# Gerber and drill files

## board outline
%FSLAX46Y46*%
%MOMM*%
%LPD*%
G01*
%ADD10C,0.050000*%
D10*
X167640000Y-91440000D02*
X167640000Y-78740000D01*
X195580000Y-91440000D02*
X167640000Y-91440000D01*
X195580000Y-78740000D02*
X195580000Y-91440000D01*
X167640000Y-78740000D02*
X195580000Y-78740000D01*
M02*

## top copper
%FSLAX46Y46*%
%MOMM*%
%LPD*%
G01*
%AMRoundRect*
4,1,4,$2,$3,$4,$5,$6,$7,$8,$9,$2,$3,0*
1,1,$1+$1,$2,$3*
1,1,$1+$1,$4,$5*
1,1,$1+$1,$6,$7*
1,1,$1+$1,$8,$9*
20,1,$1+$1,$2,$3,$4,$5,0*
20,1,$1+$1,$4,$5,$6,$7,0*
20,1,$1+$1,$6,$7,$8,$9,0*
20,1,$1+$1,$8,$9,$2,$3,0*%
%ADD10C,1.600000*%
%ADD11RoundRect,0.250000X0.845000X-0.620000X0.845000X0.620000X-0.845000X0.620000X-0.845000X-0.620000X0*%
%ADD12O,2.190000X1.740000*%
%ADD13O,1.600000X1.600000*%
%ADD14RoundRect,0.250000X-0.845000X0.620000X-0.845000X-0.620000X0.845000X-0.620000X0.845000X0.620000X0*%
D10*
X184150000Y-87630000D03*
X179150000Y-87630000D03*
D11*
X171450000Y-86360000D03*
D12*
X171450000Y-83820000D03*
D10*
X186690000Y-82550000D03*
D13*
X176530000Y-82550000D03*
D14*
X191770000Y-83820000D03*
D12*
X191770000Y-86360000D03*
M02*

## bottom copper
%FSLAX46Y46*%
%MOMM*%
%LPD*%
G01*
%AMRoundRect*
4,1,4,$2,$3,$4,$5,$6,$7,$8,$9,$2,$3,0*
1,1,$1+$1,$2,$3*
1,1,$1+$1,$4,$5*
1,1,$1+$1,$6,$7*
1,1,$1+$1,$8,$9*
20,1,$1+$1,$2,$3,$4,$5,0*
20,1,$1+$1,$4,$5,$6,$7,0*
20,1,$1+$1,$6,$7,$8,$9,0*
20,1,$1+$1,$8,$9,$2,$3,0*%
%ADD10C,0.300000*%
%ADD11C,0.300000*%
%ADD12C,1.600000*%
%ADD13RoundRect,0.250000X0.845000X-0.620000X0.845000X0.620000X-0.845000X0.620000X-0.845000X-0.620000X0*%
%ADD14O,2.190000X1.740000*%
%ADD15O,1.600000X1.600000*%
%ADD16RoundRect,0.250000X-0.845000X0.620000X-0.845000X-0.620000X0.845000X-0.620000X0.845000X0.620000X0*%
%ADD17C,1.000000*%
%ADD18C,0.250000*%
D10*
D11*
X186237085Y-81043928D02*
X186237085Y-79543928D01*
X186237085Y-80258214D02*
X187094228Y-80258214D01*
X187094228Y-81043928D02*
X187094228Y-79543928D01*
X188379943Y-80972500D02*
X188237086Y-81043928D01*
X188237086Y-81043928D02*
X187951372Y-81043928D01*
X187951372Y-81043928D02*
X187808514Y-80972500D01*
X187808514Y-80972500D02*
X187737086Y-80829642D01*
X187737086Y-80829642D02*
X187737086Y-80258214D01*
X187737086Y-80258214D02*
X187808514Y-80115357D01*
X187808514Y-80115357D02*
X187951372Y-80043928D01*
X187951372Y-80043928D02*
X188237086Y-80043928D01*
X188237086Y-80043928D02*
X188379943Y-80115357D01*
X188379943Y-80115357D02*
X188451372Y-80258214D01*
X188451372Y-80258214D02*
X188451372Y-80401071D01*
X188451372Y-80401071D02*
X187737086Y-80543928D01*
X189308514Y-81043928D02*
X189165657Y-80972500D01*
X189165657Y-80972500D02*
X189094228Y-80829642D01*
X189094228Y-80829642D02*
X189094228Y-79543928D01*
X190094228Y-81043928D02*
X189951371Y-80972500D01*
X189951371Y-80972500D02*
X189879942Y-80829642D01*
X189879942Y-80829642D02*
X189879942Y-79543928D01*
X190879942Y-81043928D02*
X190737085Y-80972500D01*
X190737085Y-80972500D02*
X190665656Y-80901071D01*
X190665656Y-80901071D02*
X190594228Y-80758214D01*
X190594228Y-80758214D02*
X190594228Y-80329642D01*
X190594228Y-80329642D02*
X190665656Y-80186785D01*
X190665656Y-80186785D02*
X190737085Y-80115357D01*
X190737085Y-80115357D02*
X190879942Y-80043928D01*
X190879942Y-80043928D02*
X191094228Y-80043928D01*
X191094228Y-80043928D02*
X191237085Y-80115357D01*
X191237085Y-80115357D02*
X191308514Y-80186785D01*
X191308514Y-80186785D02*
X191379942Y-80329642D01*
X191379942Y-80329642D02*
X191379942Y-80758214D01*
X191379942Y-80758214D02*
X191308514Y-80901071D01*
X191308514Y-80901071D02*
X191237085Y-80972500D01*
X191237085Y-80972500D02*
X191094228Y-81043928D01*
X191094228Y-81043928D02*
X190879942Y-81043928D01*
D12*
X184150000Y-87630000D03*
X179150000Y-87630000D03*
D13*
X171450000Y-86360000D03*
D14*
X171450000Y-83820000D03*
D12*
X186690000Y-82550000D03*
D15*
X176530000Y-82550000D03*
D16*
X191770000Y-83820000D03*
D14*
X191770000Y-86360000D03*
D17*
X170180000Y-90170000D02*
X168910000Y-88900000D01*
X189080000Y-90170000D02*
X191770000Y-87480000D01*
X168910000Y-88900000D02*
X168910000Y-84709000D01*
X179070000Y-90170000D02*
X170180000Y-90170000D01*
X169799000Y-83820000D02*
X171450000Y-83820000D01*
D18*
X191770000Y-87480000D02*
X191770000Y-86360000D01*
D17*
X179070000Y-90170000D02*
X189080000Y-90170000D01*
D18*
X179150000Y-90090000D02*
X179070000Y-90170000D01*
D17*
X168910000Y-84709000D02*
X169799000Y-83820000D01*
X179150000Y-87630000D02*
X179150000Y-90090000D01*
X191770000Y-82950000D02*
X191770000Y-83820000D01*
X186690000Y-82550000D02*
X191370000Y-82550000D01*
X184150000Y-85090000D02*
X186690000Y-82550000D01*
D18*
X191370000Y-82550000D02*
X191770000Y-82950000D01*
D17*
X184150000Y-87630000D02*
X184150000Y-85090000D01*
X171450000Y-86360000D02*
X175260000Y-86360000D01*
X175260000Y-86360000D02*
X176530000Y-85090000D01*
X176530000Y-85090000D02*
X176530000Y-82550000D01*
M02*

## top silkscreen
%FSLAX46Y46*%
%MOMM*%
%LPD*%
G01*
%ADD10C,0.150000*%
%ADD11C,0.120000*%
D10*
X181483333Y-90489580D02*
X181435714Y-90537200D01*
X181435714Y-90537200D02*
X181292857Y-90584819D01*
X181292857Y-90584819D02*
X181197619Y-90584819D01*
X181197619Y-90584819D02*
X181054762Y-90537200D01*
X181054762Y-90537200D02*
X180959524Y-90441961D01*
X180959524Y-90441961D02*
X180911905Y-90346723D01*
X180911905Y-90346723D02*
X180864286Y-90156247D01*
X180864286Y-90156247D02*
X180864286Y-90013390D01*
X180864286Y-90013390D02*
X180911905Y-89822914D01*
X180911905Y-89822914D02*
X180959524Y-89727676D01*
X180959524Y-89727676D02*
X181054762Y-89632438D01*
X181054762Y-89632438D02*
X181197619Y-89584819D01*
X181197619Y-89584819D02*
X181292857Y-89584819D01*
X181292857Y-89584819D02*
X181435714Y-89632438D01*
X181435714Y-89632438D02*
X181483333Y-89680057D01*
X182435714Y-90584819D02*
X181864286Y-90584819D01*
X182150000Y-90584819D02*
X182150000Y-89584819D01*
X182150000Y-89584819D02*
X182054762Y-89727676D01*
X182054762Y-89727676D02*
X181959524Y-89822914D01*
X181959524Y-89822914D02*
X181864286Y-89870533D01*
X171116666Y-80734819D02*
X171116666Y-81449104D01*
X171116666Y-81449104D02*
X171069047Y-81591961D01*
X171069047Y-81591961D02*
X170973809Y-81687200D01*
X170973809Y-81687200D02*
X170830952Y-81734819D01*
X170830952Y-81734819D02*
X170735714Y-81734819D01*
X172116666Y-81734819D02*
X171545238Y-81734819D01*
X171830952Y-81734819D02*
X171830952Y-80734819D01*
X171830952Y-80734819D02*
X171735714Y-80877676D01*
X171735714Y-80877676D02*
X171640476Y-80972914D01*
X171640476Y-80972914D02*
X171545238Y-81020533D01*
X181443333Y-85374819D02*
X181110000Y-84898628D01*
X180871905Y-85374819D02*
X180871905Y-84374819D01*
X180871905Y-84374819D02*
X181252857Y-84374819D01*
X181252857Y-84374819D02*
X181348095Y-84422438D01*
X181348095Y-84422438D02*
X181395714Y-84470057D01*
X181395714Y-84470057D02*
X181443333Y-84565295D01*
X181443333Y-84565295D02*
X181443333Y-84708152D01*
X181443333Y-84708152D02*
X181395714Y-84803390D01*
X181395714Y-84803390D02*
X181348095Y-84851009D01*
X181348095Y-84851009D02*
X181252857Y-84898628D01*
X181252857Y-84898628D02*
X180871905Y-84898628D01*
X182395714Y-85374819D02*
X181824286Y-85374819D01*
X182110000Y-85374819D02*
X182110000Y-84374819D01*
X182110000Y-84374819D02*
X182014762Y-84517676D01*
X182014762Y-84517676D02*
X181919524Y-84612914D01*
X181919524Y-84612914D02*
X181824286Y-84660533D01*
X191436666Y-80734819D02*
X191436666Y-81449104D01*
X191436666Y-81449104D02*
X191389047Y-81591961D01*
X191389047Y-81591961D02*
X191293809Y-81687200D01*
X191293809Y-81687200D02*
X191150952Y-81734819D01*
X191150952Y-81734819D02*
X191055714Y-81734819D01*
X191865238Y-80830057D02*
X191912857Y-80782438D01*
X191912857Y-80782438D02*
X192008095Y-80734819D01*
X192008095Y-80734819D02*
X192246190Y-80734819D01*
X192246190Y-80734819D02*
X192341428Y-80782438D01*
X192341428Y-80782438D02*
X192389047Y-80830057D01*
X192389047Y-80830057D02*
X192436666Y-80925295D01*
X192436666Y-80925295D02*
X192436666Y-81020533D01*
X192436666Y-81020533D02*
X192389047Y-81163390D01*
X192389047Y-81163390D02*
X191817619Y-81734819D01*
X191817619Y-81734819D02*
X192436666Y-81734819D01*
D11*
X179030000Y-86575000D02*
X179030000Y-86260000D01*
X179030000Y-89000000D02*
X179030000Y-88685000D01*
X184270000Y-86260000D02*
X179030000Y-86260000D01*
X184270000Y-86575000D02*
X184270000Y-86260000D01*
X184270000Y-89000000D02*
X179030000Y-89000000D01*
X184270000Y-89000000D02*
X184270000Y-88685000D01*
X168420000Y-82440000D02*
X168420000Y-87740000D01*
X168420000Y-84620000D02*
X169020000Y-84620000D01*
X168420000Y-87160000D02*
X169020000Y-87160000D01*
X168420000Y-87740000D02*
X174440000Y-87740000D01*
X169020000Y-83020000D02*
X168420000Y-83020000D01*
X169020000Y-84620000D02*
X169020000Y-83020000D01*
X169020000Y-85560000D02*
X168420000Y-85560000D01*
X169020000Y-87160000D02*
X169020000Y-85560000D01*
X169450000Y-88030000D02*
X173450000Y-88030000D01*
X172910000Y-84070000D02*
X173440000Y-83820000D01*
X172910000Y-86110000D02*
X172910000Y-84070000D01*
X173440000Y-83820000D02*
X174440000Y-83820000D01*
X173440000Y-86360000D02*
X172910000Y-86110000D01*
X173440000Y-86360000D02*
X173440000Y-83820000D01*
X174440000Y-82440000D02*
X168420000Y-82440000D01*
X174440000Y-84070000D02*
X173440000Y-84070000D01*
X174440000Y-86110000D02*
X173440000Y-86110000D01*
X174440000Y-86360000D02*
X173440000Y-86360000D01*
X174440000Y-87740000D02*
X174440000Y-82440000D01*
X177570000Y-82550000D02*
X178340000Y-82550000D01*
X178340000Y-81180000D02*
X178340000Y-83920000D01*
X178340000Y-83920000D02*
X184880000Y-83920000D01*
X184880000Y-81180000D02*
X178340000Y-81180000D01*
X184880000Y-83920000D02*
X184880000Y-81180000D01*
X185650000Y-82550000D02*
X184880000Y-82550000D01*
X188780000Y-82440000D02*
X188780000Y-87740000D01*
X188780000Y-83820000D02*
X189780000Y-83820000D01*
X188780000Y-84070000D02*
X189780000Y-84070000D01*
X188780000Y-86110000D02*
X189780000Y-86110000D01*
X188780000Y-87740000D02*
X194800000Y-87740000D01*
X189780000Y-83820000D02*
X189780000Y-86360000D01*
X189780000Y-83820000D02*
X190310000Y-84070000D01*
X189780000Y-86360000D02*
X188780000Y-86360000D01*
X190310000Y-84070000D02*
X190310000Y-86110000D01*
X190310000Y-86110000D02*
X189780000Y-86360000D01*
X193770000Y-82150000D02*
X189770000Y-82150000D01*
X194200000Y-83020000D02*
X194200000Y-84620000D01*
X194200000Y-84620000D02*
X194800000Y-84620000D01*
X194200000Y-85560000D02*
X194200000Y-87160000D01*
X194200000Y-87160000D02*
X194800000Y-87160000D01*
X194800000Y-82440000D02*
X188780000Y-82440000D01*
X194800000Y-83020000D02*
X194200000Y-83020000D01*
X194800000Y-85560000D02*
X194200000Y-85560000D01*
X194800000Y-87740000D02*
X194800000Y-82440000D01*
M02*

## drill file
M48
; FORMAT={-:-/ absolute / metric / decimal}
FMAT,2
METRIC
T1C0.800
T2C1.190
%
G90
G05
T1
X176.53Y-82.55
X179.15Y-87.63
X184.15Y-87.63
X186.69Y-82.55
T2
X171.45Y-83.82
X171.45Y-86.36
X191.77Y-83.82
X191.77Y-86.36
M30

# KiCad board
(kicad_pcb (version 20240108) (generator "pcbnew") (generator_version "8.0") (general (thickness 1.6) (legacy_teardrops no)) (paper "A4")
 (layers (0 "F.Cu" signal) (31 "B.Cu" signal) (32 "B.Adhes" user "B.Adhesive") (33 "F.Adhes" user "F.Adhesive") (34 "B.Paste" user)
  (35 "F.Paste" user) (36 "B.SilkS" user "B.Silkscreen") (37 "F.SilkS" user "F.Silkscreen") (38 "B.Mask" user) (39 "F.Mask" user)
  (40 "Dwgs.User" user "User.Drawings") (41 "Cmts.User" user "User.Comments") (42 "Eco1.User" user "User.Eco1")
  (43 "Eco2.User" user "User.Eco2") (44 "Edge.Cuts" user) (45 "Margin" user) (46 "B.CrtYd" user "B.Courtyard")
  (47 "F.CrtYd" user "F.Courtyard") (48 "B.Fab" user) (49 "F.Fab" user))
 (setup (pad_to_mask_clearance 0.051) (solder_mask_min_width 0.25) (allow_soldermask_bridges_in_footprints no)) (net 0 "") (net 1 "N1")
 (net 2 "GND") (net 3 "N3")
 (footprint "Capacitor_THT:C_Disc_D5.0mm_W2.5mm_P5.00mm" (layer "F.Cu") (at 184.15 87.63 180)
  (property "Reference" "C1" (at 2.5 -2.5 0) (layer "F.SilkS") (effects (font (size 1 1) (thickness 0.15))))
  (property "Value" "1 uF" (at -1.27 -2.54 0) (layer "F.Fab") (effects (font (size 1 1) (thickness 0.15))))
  (fp_line (start 5.12 1.055) (end 5.12 1.37) (stroke (width 0.12) (type solid)) (layer "F.SilkS"))
  (fp_line (start 5.12 -1.37) (end 5.12 -1.055) (stroke (width 0.12) (type solid)) (layer "F.SilkS"))
  (fp_line (start -0.12 1.37) (end 5.12 1.37) (stroke (width 0.12) (type solid)) (layer "F.SilkS"))
  (fp_line (start -0.12 1.055) (end -0.12 1.37) (stroke (width 0.12) (type solid)) (layer "F.SilkS"))
  (fp_line (start -0.12 -1.37) (end 5.12 -1.37) (stroke (width 0.12) (type solid)) (layer "F.SilkS"))
  (fp_line (start -0.12 -1.37) (end -0.12 -1.055) (stroke (width 0.12) (type solid)) (layer "F.SilkS"))
  (pad "1" thru_hole circle (at 0 0 180) (size 1.6 1.6) (drill 0.8) (layers "*.Cu" "*.Mask") (remove_unused_layers no) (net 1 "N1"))
  (pad "2" thru_hole circle (at 5 0 180) (size 1.6 1.6) (drill 0.8) (layers "*.Cu" "*.Mask") (remove_unused_layers no) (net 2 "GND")))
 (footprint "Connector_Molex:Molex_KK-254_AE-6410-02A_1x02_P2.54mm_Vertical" (layer "F.Cu") (at 171.45 86.36 90)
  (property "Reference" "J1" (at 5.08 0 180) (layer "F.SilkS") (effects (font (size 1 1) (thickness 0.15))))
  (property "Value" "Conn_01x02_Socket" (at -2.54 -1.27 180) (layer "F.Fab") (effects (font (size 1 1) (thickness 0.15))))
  (fp_line (start 3.92 -3.03) (end -1.38 -3.03) (stroke (width 0.12) (type solid)) (layer "F.SilkS"))
  (fp_line (start 1.74 -3.03) (end 1.74 -2.43) (stroke (width 0.12) (type solid)) (layer "F.SilkS"))
  (fp_line (start -0.8 -3.03) (end -0.8 -2.43) (stroke (width 0.12) (type solid)) (layer "F.SilkS"))
  (fp_line (start -1.38 -3.03) (end -1.38 2.99) (stroke (width 0.12) (type solid)) (layer "F.SilkS"))
  (fp_line (start 3.34 -2.43) (end 3.34 -3.03) (stroke (width 0.12) (type solid)) (layer "F.SilkS"))
  (fp_line (start 1.74 -2.43) (end 3.34 -2.43) (stroke (width 0.12) (type solid)) (layer "F.SilkS"))
  (fp_line (start 0.8 -2.43) (end 0.8 -3.03) (stroke (width 0.12) (type solid)) (layer "F.SilkS"))
  (fp_line (start -0.8 -2.43) (end 0.8 -2.43) (stroke (width 0.12) (type solid)) (layer "F.SilkS"))
  (fp_line (start -1.67 -2) (end -1.67 2) (stroke (width 0.12) (type solid)) (layer "F.SilkS"))
  (fp_line (start 2.29 1.46) (end 2.54 1.99) (stroke (width 0.12) (type solid)) (layer "F.SilkS"))
  (fp_line (start 0.25 1.46) (end 2.29 1.46) (stroke (width 0.12) (type solid)) (layer "F.SilkS"))
  (fp_line (start 2.54 1.99) (end 2.54 2.99) (stroke (width 0.12) (type solid)) (layer "F.SilkS"))
  (fp_line (start 0 1.99) (end 0.25 1.46) (stroke (width 0.12) (type solid)) (layer "F.SilkS"))
  (fp_line (start 0 1.99) (end 2.54 1.99) (stroke (width 0.12) (type solid)) (layer "F.SilkS"))
  (fp_line (start 3.92 2.99) (end 3.92 -3.03) (stroke (width 0.12) (type solid)) (layer "F.SilkS"))
  (fp_line (start 2.29 2.99) (end 2.29 1.99) (stroke (width 0.12) (type solid)) (layer "F.SilkS"))
  (fp_line (start 0.25 2.99) (end 0.25 1.99) (stroke (width 0.12) (type solid)) (layer "F.SilkS"))
  (fp_line (start 0 2.99) (end 0 1.99) (stroke (width 0.12) (type solid)) (layer "F.SilkS"))
  (fp_line (start -1.38 2.99) (end 3.92 2.99) (stroke (width 0.12) (type solid)) (layer "F.SilkS"))
  (pad "1" thru_hole roundrect (at 0 0 90) (size 1.74 2.19) (drill 1.19) (layers "*.Cu" "*.Mask") (remove_unused_layers no)
   (roundrect_rratio 0.143678) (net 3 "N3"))
  (pad "2" thru_hole oval (at 2.54 0 90) (size 1.74 2.19) (drill 1.19) (layers "*.Cu" "*.Mask") (remove_unused_layers no) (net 2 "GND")))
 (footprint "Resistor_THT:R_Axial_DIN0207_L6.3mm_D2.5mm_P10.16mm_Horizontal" (layer "F.Cu") (at 186.69 82.55 180)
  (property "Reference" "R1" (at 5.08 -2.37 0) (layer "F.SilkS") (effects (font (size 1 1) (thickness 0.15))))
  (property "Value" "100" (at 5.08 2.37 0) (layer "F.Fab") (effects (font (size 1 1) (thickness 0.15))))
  (fp_line (start 9.12 0) (end 8.35 0) (stroke (width 0.12) (type solid)) (layer "F.SilkS"))
  (fp_line (start 8.35 1.37) (end 8.35 -1.37) (stroke (width 0.12) (type solid)) (layer "F.SilkS"))
  (fp_line (start 8.35 -1.37) (end 1.81 -1.37) (stroke (width 0.12) (type solid)) (layer "F.SilkS"))
  (fp_line (start 1.81 1.37) (end 8.35 1.37) (stroke (width 0.12) (type solid)) (layer "F.SilkS"))
  (fp_line (start 1.81 -1.37) (end 1.81 1.37) (stroke (width 0.12) (type solid)) (layer "F.SilkS"))
  (fp_line (start 1.04 0) (end 1.81 0) (stroke (width 0.12) (type solid)) (layer "F.SilkS"))
  (pad "1" thru_hole circle (at 0 0 180) (size 1.6 1.6) (drill 0.8) (layers "*.Cu" "*.Mask") (remove_unused_layers no) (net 1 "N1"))
  (pad "2" thru_hole oval (at 10.16 0 180) (size 1.6 1.6) (drill 0.8) (layers "*.Cu" "*.Mask") (remove_unused_layers no) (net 3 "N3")))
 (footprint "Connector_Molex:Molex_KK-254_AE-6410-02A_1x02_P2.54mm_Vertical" (layer "F.Cu") (at 191.77 83.82 -90)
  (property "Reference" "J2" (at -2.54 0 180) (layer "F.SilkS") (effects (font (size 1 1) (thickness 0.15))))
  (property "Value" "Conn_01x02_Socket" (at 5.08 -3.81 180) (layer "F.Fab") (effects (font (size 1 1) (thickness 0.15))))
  (fp_line (start -1.38 2.99) (end 3.92 2.99) (stroke (width 0.12) (type solid)) (layer "F.SilkS"))
  (fp_line (start 0 2.99) (end 0 1.99) (stroke (width 0.12) (type solid)) (layer "F.SilkS"))
  (fp_line (start 0.25 2.99) (end 0.25 1.99) (stroke (width 0.12) (type solid)) (layer "F.SilkS"))
  (fp_line (start 2.29 2.99) (end 2.29 1.99) (stroke (width 0.12) (type solid)) (layer "F.SilkS"))
  (fp_line (start 3.92 2.99) (end 3.92 -3.03) (stroke (width 0.12) (type solid)) (layer "F.SilkS"))
  (fp_line (start 0 1.99) (end 2.54 1.99) (stroke (width 0.12) (type solid)) (layer "F.SilkS"))
  (fp_line (start 0 1.99) (end 0.25 1.46) (stroke (width 0.12) (type solid)) (layer "F.SilkS"))
  (fp_line (start 2.54 1.99) (end 2.54 2.99) (stroke (width 0.12) (type solid)) (layer "F.SilkS"))
  (fp_line (start 0.25 1.46) (end 2.29 1.46) (stroke (width 0.12) (type solid)) (layer "F.SilkS"))
  (fp_line (start 2.29 1.46) (end 2.54 1.99) (stroke (width 0.12) (type solid)) (layer "F.SilkS"))
  (fp_line (start -1.67 -2) (end -1.67 2) (stroke (width 0.12) (type solid)) (layer "F.SilkS"))
  (fp_line (start -0.8 -2.43) (end 0.8 -2.43) (stroke (width 0.12) (type solid)) (layer "F.SilkS"))
  (fp_line (start 0.8 -2.43) (end 0.8 -3.03) (stroke (width 0.12) (type solid)) (layer "F.SilkS"))
  (fp_line (start 1.74 -2.43) (end 3.34 -2.43) (stroke (width 0.12) (type solid)) (layer "F.SilkS"))
  (fp_line (start 3.34 -2.43) (end 3.34 -3.03) (stroke (width 0.12) (type solid)) (layer "F.SilkS"))
  (fp_line (start -1.38 -3.03) (end -1.38 2.99) (stroke (width 0.12) (type solid)) (layer "F.SilkS"))
  (fp_line (start -0.8 -3.03) (end -0.8 -2.43) (stroke (width 0.12) (type solid)) (layer "F.SilkS"))
  (fp_line (start 1.74 -3.03) (end 1.74 -2.43) (stroke (width 0.12) (type solid)) (layer "F.SilkS"))
  (fp_line (start 3.92 -3.03) (end -1.38 -3.03) (stroke (width 0.12) (type solid)) (layer "F.SilkS"))
  (pad "1" thru_hole roundrect (at 0 0 270) (size 1.74 2.19) (drill 1.19) (layers "*.Cu" "*.Mask") (remove_unused_layers no)
   (roundrect_rratio 0.143678) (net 1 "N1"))
  (pad "2" thru_hole oval (at 2.54 0 270) (size 1.74 2.19) (drill 1.19) (layers "*.Cu" "*.Mask") (remove_unused_layers no) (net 2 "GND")))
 (gr_line (start 167.64 91.44) (end 167.64 78.74) (stroke (width 0.05) (type solid)) (layer "Edge.Cuts"))
 (gr_line (start 195.58 91.44) (end 167.64 91.44) (stroke (width 0.05) (type solid)) (layer "Edge.Cuts"))
 (gr_line (start 195.58 78.74) (end 195.58 91.44) (stroke (width 0.05) (type solid)) (layer "Edge.Cuts"))
 (gr_line (start 167.64 78.74) (end 195.58 78.74) (stroke (width 0.05) (type solid)) (layer "Edge.Cuts"))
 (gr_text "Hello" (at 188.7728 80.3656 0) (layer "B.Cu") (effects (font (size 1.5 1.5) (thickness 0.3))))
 (segment (start 170.18 90.17) (end 168.91 88.9) (width 1) (layer "B.Cu") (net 2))
 (segment (start 189.08 90.17) (end 191.77 87.48) (width 1) (layer "B.Cu") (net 2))
 (segment (start 168.91 88.9) (end 168.91 84.709) (width 1) (layer "B.Cu") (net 2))
 (segment (start 179.07 90.17) (end 170.18 90.17) (width 1) (layer "B.Cu") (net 2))
 (segment (start 169.799 83.82) (end 171.45 83.82) (width 1) (layer "B.Cu") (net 2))
 (segment (start 191.77 87.48) (end 191.77 86.36) (width 0.25) (layer "B.Cu") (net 2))
 (segment (start 179.07 90.17) (end 189.08 90.17) (width 1) (layer "B.Cu") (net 2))
 (segment (start 179.15 90.09) (end 179.07 90.17) (width 0.25) (layer "B.Cu") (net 2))
 (segment (start 168.91 84.709) (end 169.799 83.82) (width 1) (layer "B.Cu") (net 2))
 (segment (start 179.15 87.63) (end 179.15 90.09) (width 1) (layer "B.Cu") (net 2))
 (segment (start 191.77 82.95) (end 191.77 83.82) (width 1) (layer "B.Cu") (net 1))
 (segment (start 186.69 82.55) (end 191.37 82.55) (width 1) (layer "B.Cu") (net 1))
 (segment (start 184.15 85.09) (end 186.69 82.55) (width 1) (layer "B.Cu") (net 1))
 (segment (start 191.37 82.55) (end 191.77 82.95) (width 0.25) (layer "B.Cu") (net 1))
 (segment (start 184.15 87.63) (end 184.15 85.09) (width 1) (layer "B.Cu") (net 1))
 (segment (start 171.45 86.36) (end 175.26 86.36) (width 1) (layer "B.Cu") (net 3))
 (segment (start 175.26 86.36) (end 176.53 85.09) (width 1) (layer "B.Cu") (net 3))
 (segment (start 176.53 85.09) (end 176.53 82.55) (width 1) (layer "B.Cu") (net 3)))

